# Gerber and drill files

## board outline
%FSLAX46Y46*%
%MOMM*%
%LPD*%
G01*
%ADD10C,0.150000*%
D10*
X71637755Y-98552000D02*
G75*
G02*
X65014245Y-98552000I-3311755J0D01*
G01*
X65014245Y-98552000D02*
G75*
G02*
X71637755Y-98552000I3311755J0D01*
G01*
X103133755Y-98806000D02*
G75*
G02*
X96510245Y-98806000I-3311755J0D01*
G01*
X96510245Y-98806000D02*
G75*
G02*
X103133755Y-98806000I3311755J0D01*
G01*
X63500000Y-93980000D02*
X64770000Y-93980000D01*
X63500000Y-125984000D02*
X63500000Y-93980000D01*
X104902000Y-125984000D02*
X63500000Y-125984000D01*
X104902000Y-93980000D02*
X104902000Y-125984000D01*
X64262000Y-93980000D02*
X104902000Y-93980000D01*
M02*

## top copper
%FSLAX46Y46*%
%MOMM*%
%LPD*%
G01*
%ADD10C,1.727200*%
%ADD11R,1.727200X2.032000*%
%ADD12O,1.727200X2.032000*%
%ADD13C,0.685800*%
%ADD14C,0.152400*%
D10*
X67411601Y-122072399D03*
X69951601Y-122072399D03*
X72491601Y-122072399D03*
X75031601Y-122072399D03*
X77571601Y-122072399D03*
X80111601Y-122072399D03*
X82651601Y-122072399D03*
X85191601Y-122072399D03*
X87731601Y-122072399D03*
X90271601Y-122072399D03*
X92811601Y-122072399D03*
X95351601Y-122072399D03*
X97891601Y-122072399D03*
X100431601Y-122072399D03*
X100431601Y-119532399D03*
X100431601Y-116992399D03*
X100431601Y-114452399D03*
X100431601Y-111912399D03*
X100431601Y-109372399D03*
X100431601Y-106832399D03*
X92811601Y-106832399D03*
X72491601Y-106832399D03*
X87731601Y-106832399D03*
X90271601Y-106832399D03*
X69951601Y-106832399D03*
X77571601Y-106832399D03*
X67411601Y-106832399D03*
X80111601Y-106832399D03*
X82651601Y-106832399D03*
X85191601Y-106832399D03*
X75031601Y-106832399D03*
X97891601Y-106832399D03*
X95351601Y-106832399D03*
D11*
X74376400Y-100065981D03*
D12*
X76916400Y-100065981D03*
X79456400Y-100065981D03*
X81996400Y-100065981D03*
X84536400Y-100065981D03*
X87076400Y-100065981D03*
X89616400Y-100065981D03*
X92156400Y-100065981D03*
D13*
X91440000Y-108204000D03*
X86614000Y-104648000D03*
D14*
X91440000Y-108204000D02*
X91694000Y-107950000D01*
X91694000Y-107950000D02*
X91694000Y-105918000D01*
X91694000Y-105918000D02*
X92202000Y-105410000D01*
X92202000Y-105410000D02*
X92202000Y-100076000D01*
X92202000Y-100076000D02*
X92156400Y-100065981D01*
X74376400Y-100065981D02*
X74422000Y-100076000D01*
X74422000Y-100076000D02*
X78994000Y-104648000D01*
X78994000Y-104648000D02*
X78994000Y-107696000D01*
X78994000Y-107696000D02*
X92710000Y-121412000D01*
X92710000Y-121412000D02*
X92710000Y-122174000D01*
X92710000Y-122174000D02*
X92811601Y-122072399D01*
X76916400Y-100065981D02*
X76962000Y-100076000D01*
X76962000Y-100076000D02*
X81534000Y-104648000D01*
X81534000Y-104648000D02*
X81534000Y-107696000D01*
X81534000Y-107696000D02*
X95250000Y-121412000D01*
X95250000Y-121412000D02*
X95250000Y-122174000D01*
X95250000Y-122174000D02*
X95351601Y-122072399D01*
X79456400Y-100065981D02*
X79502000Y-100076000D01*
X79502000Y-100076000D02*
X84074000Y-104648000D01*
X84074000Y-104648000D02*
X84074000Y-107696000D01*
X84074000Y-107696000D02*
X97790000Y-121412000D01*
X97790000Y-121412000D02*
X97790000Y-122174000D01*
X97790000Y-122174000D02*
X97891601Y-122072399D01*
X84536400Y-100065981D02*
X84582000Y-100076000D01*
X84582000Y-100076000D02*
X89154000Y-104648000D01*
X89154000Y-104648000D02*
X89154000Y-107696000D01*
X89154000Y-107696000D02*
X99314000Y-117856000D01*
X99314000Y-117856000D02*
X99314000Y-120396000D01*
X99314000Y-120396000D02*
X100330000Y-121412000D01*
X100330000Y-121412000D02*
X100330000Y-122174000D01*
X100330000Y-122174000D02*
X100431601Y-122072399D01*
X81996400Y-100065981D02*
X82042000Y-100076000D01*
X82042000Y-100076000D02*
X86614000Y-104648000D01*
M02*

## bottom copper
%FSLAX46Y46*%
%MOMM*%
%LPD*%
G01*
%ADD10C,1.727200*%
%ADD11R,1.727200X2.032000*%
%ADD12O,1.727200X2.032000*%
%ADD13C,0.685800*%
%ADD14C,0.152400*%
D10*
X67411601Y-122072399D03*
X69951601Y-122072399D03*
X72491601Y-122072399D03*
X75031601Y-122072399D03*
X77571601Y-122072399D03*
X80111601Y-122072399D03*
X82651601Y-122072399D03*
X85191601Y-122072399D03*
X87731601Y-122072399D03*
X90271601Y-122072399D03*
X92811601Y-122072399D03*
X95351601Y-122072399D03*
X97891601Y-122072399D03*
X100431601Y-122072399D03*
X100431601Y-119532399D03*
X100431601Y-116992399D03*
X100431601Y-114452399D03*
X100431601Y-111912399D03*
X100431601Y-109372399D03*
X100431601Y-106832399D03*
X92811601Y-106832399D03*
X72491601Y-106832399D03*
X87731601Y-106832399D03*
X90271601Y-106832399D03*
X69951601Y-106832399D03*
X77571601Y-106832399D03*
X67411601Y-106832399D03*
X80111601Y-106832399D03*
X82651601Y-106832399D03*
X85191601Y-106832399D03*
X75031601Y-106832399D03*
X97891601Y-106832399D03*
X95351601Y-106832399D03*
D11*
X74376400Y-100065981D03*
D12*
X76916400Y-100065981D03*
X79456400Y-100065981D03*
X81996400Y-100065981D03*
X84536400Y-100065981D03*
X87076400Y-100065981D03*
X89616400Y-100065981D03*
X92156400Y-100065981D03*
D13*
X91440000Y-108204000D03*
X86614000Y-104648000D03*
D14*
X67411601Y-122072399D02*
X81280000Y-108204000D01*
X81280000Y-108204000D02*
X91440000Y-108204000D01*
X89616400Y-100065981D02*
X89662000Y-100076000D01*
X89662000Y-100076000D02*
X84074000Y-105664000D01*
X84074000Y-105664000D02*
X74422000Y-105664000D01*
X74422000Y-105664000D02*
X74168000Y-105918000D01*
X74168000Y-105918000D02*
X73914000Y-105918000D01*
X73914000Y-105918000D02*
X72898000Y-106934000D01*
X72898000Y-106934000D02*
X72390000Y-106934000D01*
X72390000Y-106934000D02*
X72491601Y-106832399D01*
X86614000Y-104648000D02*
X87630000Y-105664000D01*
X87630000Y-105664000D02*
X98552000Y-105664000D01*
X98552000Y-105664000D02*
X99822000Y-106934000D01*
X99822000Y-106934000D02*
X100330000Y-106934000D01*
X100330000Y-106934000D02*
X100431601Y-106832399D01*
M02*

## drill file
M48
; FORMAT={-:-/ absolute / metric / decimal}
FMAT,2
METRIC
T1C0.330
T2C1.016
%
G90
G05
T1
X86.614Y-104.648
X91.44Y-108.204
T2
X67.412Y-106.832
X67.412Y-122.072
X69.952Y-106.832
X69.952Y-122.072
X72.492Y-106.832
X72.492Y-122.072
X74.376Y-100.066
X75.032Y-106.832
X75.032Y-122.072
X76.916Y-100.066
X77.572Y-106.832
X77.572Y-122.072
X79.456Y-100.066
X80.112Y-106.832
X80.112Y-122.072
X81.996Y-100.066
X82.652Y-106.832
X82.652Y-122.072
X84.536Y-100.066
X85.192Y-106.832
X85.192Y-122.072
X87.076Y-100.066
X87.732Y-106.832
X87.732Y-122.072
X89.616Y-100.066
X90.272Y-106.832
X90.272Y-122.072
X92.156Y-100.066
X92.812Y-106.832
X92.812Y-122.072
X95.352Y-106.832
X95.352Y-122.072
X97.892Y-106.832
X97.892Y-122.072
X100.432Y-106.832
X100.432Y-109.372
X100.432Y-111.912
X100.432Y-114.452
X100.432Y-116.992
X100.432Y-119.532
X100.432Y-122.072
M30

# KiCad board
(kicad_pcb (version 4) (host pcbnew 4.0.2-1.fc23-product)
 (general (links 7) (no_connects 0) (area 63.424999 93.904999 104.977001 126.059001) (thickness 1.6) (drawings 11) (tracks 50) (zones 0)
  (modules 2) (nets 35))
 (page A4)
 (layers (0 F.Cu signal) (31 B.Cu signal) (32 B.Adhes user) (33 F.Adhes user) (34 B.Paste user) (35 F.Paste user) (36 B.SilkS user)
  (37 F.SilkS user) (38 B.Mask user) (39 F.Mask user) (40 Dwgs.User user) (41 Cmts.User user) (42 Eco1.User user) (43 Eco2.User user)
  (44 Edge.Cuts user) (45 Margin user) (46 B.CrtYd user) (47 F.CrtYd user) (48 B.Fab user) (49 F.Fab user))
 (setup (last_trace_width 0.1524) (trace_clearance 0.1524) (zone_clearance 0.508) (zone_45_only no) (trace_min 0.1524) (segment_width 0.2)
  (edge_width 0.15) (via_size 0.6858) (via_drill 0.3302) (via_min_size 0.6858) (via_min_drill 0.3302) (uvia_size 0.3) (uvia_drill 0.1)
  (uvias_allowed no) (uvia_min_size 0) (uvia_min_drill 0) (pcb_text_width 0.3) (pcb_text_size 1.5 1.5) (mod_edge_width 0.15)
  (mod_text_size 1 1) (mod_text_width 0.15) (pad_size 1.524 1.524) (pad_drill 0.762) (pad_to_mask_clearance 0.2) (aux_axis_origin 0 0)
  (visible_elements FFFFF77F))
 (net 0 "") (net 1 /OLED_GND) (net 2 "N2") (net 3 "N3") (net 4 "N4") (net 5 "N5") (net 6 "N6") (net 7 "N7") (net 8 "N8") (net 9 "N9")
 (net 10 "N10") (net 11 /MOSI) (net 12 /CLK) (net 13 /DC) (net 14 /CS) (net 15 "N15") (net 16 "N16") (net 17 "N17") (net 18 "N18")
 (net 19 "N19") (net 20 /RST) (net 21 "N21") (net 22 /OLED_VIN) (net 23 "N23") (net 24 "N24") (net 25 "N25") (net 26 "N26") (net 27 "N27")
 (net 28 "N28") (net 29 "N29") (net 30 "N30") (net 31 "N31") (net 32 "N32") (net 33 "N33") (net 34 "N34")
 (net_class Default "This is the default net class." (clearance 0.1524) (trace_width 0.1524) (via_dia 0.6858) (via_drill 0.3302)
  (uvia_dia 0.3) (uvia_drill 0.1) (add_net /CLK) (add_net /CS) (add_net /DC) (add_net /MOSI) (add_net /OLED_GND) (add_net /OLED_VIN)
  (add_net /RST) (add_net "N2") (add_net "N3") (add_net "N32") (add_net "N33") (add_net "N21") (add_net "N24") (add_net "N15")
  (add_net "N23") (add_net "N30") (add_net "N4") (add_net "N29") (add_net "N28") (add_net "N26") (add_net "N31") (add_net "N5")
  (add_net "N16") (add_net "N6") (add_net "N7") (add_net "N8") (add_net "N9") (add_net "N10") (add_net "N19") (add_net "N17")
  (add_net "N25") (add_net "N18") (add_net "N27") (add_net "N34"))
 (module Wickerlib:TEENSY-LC (layer F.Cu) (at 77.571601 111.912399 90)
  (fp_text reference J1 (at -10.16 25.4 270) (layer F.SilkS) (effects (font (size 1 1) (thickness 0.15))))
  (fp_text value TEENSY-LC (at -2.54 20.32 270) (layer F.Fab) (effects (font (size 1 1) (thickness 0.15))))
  (pad G1 thru_hole circle (at -10.16 -10.16 90) (size 1.7272 1.7272) (drill 1.016) (layers *.Cu *.Mask F.SilkS) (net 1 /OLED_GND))
  (pad 0 thru_hole circle (at -10.16 -7.62 90) (size 1.7272 1.7272) (drill 1.016) (layers *.Cu *.Mask F.SilkS) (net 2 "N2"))
  (pad 1 thru_hole circle (at -10.16 -5.08 90) (size 1.7272 1.7272) (drill 1.016) (layers *.Cu *.Mask F.SilkS) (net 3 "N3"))
  (pad 2 thru_hole circle (at -10.16 -2.54 90) (size 1.7272 1.7272) (drill 1.016) (layers *.Cu *.Mask F.SilkS) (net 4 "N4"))
  (pad 3 thru_hole circle (at -10.16 0 90) (size 1.7272 1.7272) (drill 1.016) (layers *.Cu *.Mask F.SilkS) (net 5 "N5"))
  (pad 4 thru_hole circle (at -10.16 2.54 90) (size 1.7272 1.7272) (drill 1.016) (layers *.Cu *.Mask F.SilkS) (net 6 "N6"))
  (pad 5 thru_hole circle (at -10.16 5.08 90) (size 1.7272 1.7272) (drill 1.016) (layers *.Cu *.Mask F.SilkS) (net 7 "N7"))
  (pad 6 thru_hole circle (at -10.16 7.62 90) (size 1.7272 1.7272) (drill 1.016) (layers *.Cu *.Mask F.SilkS) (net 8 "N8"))
  (pad 7 thru_hole circle (at -10.16 10.16 90) (size 1.7272 1.7272) (drill 1.016) (layers *.Cu *.Mask F.SilkS) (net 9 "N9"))
  (pad 8 thru_hole circle (at -10.16 12.7 90) (size 1.7272 1.7272) (drill 1.016) (layers *.Cu *.Mask F.SilkS) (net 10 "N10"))
  (pad 9 thru_hole circle (at -10.16 15.24 90) (size 1.7272 1.7272) (drill 1.016) (layers *.Cu *.Mask F.SilkS) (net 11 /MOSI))
  (pad 10 thru_hole circle (at -10.16 17.78 90) (size 1.7272 1.7272) (drill 1.016) (layers *.Cu *.Mask F.SilkS) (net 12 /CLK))
  (pad 11 thru_hole circle (at -10.16 20.32 90) (size 1.7272 1.7272) (drill 1.016) (layers *.Cu *.Mask F.SilkS) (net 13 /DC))
  (pad 12 thru_hole circle (at -10.16 22.86 90) (size 1.7272 1.7272) (drill 1.016) (layers *.Cu *.Mask F.SilkS) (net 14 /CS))
  (pad 17A thru_hole circle (at -7.62 22.86 90) (size 1.7272 1.7272) (drill 1.016) (layers *.Cu *.Mask F.SilkS) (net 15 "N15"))
  (pad 3V1 thru_hole circle (at -5.08 22.86 90) (size 1.7272 1.7272) (drill 1.016) (layers *.Cu *.Mask F.SilkS) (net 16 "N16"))
  (pad G2 thru_hole circle (at -2.54 22.86 90) (size 1.7272 1.7272) (drill 1.016) (layers *.Cu *.Mask F.SilkS) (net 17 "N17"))
  (pad PGM thru_hole circle (at 0 22.86 90) (size 1.7272 1.7272) (drill 1.016) (layers *.Cu *.Mask F.SilkS) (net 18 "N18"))
  (pad DAC thru_hole circle (at 2.54 22.86 90) (size 1.7272 1.7272) (drill 1.016) (layers *.Cu *.Mask F.SilkS) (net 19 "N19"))
  (pad 13 thru_hole circle (at 5.08 22.86 90) (size 1.7272 1.7272) (drill 1.016) (layers *.Cu *.Mask F.SilkS) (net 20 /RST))
  (pad 16 thru_hole circle (at 5.08 15.24 90) (size 1.7272 1.7272) (drill 1.016) (layers *.Cu *.Mask F.SilkS) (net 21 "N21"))
  (pad 3V2 thru_hole circle (at 5.08 -5.08 90) (size 1.7272 1.7272) (drill 1.016) (layers *.Cu *.Mask F.SilkS) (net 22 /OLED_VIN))
  (pad 18 thru_hole circle (at 5.08 10.16 90) (size 1.7272 1.7272) (drill 1.016) (layers *.Cu *.Mask F.SilkS) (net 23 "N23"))
  (pad 17 thru_hole circle (at 5.08 12.7 90) (size 1.7272 1.7272) (drill 1.016) (layers *.Cu *.Mask F.SilkS) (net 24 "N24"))
  (pad G3 thru_hole circle (at 5.08 -7.62 90) (size 1.7272 1.7272) (drill 1.016) (layers *.Cu *.Mask F.SilkS) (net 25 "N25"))
  (pad 22 thru_hole circle (at 5.08 0 90) (size 1.7272 1.7272) (drill 1.016) (layers *.Cu *.Mask F.SilkS) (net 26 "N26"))
  (pad VIN thru_hole circle (at 5.08 -10.16 90) (size 1.7272 1.7272) (drill 1.016) (layers *.Cu *.Mask F.SilkS) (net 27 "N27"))
  (pad 21 thru_hole circle (at 5.08 2.54 90) (size 1.7272 1.7272) (drill 1.016) (layers *.Cu *.Mask F.SilkS) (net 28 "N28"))
  (pad 20 thru_hole circle (at 5.08 5.08 90) (size 1.7272 1.7272) (drill 1.016) (layers *.Cu *.Mask F.SilkS) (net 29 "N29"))
  (pad 19 thru_hole circle (at 5.08 7.62 90) (size 1.7272 1.7272) (drill 1.016) (layers *.Cu *.Mask F.SilkS) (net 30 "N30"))
  (pad 23 thru_hole circle (at 5.08 -2.54 90) (size 1.7272 1.7272) (drill 1.016) (layers *.Cu *.Mask F.SilkS) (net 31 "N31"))
  (pad 14 thru_hole circle (at 5.08 20.32 90) (size 1.7272 1.7272) (drill 1.016) (layers *.Cu *.Mask F.SilkS) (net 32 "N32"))
  (pad 15 thru_hole circle (at 5.08 17.78 90) (size 1.7272 1.7272) (drill 1.016) (layers *.Cu *.Mask F.SilkS) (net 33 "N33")))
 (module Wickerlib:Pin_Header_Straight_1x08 (layer F.Cu) (at 74.3764 100.065981 90)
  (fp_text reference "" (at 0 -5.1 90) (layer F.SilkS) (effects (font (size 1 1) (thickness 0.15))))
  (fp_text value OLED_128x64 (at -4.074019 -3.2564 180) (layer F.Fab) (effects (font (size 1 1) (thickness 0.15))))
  (pad 1 thru_hole rect (at 0 0 90) (size 2.032 1.7272) (drill 1.016) (layers *.Cu *.Mask F.SilkS) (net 11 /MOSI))
  (pad 2 thru_hole oval (at 0 2.54 90) (size 2.032 1.7272) (drill 1.016) (layers *.Cu *.Mask F.SilkS) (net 12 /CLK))
  (pad 3 thru_hole oval (at 0 5.08 90) (size 2.032 1.7272) (drill 1.016) (layers *.Cu *.Mask F.SilkS) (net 13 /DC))
  (pad 4 thru_hole oval (at 0 7.62 90) (size 2.032 1.7272) (drill 1.016) (layers *.Cu *.Mask F.SilkS) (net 20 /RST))
  (pad 5 thru_hole oval (at 0 10.16 90) (size 2.032 1.7272) (drill 1.016) (layers *.Cu *.Mask F.SilkS) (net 14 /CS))
  (pad 6 thru_hole oval (at 0 12.7 90) (size 2.032 1.7272) (drill 1.016) (layers *.Cu *.Mask F.SilkS) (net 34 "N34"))
  (pad 7 thru_hole oval (at 0 15.24 90) (size 2.032 1.7272) (drill 1.016) (layers *.Cu *.Mask F.SilkS) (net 22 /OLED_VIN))
  (pad 8 thru_hole oval (at 0 17.78 90) (size 2.032 1.7272) (drill 1.016) (layers *.Cu *.Mask F.SilkS) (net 1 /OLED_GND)))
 (gr_circle (center 68.326 98.552) (end 65.532 96.774) (layer Edge.Cuts) (width 0.15))
 (gr_circle (center 99.822 98.806) (end 97.028 97.028) (layer Edge.Cuts) (width 0.15))
 (gr_line (start 63.5 93.98) (end 64.77 93.98) (angle 90) (layer Edge.Cuts) (width 0.15))
 (gr_line (start 63.5 125.984) (end 63.5 93.98) (angle 90) (layer Edge.Cuts) (width 0.15))
 (gr_line (start 104.902 125.984) (end 63.5 125.984) (angle 90) (layer Edge.Cuts) (width 0.15))
 (gr_line (start 104.902 93.98) (end 104.902 125.984) (angle 90) (layer Edge.Cuts) (width 0.15))
 (gr_line (start 64.262 93.98) (end 104.902 93.98) (angle 90) (layer Edge.Cuts) (width 0.15))
 (segment (start 67.411601 122.072399) (end 81.28 108.204) (width 0.1524) (layer B.Cu) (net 1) (status 80000))
 (segment (start 81.28 108.204) (end 91.44 108.204) (width 0.1524) (layer B.Cu) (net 1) (status 80000))
 (via (at 91.44 108.204) (size 0.6858) (layers F.Cu B.Cu) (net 1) (status 80000))
 (segment (start 91.44 108.204) (end 91.694 107.95) (width 0.1524) (layer F.Cu) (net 1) (status 80000))
 (segment (start 91.694 107.95) (end 91.694 105.918) (width 0.1524) (layer F.Cu) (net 1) (status 80000))
 (segment (start 91.694 105.918) (end 92.202 105.41) (width 0.1524) (layer F.Cu) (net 1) (status 80000))
 (segment (start 92.202 105.41) (end 92.202 100.076) (width 0.1524) (layer F.Cu) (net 1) (status 80000))
 (segment (start 92.202 100.076) (end 92.1564 100.065981) (width 0.1524) (layer F.Cu) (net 1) (status 80000))
 (segment (start 74.3764 100.065981) (end 74.422 100.076) (width 0.1524) (layer F.Cu) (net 11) (status 80000))
 (segment (start 74.422 100.076) (end 78.994 104.648) (width 0.1524) (layer F.Cu) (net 11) (status 80000))
 (segment (start 78.994 104.648) (end 78.994 107.696) (width 0.1524) (layer F.Cu) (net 11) (status 80000))
 (segment (start 78.994 107.696) (end 92.71 121.412) (width 0.1524) (layer F.Cu) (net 11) (status 80000))
 (segment (start 92.71 121.412) (end 92.71 122.174) (width 0.1524) (layer F.Cu) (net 11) (status 80000))
 (segment (start 92.71 122.174) (end 92.811601 122.072399) (width 0.1524) (layer F.Cu) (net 11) (status 80000))
 (segment (start 76.9164 100.065981) (end 76.962 100.076) (width 0.1524) (layer F.Cu) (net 12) (status 80000))
 (segment (start 76.962 100.076) (end 81.534 104.648) (width 0.1524) (layer F.Cu) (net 12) (status 80000))
 (segment (start 81.534 104.648) (end 81.534 107.696) (width 0.1524) (layer F.Cu) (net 12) (status 80000))
 (segment (start 81.534 107.696) (end 95.25 121.412) (width 0.1524) (layer F.Cu) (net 12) (status 80000))
 (segment (start 95.25 121.412) (end 95.25 122.174) (width 0.1524) (layer F.Cu) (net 12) (status 80000))
 (segment (start 95.25 122.174) (end 95.351601 122.072399) (width 0.1524) (layer F.Cu) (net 12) (status 80000))
 (segment (start 79.4564 100.065981) (end 79.502 100.076) (width 0.1524) (layer F.Cu) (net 13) (status 80000))
 (segment (start 79.502 100.076) (end 84.074 104.648) (width 0.1524) (layer F.Cu) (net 13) (status 80000))
 (segment (start 84.074 104.648) (end 84.074 107.696) (width 0.1524) (layer F.Cu) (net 13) (status 80000))
 (segment (start 84.074 107.696) (end 97.79 121.412) (width 0.1524) (layer F.Cu) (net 13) (status 80000))
 (segment (start 97.79 121.412) (end 97.79 122.174) (width 0.1524) (layer F.Cu) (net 13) (status 80000))
 (segment (start 97.79 122.174) (end 97.891601 122.072399) (width 0.1524) (layer F.Cu) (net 13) (status 80000))
 (segment (start 84.5364 100.065981) (end 84.582 100.076) (width 0.1524) (layer F.Cu) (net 14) (status 80000))
 (segment (start 84.582 100.076) (end 89.154 104.648) (width 0.1524) (layer F.Cu) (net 14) (status 80000))
 (segment (start 89.154 104.648) (end 89.154 107.696) (width 0.1524) (layer F.Cu) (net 14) (status 80000))
 (segment (start 89.154 107.696) (end 99.314 117.856) (width 0.1524) (layer F.Cu) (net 14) (status 80000))
 (segment (start 99.314 117.856) (end 99.314 120.396) (width 0.1524) (layer F.Cu) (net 14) (status 80000))
 (segment (start 99.314 120.396) (end 100.33 121.412) (width 0.1524) (layer F.Cu) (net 14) (status 80000))
 (segment (start 100.33 121.412) (end 100.33 122.174) (width 0.1524) (layer F.Cu) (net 14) (status 80000))
 (segment (start 100.33 122.174) (end 100.431601 122.072399) (width 0.1524) (layer F.Cu) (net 14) (status 80000))
 (segment (start 89.6164 100.065981) (end 89.662 100.076) (width 0.1524) (layer B.Cu) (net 22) (status 80000))
 (segment (start 89.662 100.076) (end 84.074 105.664) (width 0.1524) (layer B.Cu) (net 22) (status 80000))
 (segment (start 84.074 105.664) (end 74.422 105.664) (width 0.1524) (layer B.Cu) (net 22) (status 80000))
 (segment (start 74.422 105.664) (end 74.168 105.918) (width 0.1524) (layer B.Cu) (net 22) (status 80000))
 (segment (start 74.168 105.918) (end 73.914 105.918) (width 0.1524) (layer B.Cu) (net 22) (status 80000))
 (segment (start 73.914 105.918) (end 72.898 106.934) (width 0.1524) (layer B.Cu) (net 22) (status 80000))
 (segment (start 72.898 106.934) (end 72.39 106.934) (width 0.1524) (layer B.Cu) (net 22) (status 80000))
 (segment (start 72.39 106.934) (end 72.491601 106.832399) (width 0.1524) (layer B.Cu) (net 22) (status 80000))
 (segment (start 81.9964 100.065981) (end 82.042 100.076) (width 0.1524) (layer F.Cu) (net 20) (status 80000))
 (segment (start 82.042 100.076) (end 86.614 104.648) (width 0.1524) (layer F.Cu) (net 20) (status 80000))
 (via (at 86.614 104.648) (size 0.6858) (layers F.Cu B.Cu) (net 20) (status 80000))
 (segment (start 86.614 104.648) (end 87.63 105.664) (width 0.1524) (layer B.Cu) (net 20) (status 80000))
 (segment (start 87.63 105.664) (end 98.552 105.664) (width 0.1524) (layer B.Cu) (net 20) (status 80000))
 (segment (start 98.552 105.664) (end 99.822 106.934) (width 0.1524) (layer B.Cu) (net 20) (status 80000))
 (segment (start 99.822 106.934) (end 100.33 106.934) (width 0.1524) (layer B.Cu) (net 20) (status 80000))
 (segment (start 100.33 106.934) (end 100.431601 106.832399) (width 0.1524) (layer B.Cu) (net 20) (status 80000)))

